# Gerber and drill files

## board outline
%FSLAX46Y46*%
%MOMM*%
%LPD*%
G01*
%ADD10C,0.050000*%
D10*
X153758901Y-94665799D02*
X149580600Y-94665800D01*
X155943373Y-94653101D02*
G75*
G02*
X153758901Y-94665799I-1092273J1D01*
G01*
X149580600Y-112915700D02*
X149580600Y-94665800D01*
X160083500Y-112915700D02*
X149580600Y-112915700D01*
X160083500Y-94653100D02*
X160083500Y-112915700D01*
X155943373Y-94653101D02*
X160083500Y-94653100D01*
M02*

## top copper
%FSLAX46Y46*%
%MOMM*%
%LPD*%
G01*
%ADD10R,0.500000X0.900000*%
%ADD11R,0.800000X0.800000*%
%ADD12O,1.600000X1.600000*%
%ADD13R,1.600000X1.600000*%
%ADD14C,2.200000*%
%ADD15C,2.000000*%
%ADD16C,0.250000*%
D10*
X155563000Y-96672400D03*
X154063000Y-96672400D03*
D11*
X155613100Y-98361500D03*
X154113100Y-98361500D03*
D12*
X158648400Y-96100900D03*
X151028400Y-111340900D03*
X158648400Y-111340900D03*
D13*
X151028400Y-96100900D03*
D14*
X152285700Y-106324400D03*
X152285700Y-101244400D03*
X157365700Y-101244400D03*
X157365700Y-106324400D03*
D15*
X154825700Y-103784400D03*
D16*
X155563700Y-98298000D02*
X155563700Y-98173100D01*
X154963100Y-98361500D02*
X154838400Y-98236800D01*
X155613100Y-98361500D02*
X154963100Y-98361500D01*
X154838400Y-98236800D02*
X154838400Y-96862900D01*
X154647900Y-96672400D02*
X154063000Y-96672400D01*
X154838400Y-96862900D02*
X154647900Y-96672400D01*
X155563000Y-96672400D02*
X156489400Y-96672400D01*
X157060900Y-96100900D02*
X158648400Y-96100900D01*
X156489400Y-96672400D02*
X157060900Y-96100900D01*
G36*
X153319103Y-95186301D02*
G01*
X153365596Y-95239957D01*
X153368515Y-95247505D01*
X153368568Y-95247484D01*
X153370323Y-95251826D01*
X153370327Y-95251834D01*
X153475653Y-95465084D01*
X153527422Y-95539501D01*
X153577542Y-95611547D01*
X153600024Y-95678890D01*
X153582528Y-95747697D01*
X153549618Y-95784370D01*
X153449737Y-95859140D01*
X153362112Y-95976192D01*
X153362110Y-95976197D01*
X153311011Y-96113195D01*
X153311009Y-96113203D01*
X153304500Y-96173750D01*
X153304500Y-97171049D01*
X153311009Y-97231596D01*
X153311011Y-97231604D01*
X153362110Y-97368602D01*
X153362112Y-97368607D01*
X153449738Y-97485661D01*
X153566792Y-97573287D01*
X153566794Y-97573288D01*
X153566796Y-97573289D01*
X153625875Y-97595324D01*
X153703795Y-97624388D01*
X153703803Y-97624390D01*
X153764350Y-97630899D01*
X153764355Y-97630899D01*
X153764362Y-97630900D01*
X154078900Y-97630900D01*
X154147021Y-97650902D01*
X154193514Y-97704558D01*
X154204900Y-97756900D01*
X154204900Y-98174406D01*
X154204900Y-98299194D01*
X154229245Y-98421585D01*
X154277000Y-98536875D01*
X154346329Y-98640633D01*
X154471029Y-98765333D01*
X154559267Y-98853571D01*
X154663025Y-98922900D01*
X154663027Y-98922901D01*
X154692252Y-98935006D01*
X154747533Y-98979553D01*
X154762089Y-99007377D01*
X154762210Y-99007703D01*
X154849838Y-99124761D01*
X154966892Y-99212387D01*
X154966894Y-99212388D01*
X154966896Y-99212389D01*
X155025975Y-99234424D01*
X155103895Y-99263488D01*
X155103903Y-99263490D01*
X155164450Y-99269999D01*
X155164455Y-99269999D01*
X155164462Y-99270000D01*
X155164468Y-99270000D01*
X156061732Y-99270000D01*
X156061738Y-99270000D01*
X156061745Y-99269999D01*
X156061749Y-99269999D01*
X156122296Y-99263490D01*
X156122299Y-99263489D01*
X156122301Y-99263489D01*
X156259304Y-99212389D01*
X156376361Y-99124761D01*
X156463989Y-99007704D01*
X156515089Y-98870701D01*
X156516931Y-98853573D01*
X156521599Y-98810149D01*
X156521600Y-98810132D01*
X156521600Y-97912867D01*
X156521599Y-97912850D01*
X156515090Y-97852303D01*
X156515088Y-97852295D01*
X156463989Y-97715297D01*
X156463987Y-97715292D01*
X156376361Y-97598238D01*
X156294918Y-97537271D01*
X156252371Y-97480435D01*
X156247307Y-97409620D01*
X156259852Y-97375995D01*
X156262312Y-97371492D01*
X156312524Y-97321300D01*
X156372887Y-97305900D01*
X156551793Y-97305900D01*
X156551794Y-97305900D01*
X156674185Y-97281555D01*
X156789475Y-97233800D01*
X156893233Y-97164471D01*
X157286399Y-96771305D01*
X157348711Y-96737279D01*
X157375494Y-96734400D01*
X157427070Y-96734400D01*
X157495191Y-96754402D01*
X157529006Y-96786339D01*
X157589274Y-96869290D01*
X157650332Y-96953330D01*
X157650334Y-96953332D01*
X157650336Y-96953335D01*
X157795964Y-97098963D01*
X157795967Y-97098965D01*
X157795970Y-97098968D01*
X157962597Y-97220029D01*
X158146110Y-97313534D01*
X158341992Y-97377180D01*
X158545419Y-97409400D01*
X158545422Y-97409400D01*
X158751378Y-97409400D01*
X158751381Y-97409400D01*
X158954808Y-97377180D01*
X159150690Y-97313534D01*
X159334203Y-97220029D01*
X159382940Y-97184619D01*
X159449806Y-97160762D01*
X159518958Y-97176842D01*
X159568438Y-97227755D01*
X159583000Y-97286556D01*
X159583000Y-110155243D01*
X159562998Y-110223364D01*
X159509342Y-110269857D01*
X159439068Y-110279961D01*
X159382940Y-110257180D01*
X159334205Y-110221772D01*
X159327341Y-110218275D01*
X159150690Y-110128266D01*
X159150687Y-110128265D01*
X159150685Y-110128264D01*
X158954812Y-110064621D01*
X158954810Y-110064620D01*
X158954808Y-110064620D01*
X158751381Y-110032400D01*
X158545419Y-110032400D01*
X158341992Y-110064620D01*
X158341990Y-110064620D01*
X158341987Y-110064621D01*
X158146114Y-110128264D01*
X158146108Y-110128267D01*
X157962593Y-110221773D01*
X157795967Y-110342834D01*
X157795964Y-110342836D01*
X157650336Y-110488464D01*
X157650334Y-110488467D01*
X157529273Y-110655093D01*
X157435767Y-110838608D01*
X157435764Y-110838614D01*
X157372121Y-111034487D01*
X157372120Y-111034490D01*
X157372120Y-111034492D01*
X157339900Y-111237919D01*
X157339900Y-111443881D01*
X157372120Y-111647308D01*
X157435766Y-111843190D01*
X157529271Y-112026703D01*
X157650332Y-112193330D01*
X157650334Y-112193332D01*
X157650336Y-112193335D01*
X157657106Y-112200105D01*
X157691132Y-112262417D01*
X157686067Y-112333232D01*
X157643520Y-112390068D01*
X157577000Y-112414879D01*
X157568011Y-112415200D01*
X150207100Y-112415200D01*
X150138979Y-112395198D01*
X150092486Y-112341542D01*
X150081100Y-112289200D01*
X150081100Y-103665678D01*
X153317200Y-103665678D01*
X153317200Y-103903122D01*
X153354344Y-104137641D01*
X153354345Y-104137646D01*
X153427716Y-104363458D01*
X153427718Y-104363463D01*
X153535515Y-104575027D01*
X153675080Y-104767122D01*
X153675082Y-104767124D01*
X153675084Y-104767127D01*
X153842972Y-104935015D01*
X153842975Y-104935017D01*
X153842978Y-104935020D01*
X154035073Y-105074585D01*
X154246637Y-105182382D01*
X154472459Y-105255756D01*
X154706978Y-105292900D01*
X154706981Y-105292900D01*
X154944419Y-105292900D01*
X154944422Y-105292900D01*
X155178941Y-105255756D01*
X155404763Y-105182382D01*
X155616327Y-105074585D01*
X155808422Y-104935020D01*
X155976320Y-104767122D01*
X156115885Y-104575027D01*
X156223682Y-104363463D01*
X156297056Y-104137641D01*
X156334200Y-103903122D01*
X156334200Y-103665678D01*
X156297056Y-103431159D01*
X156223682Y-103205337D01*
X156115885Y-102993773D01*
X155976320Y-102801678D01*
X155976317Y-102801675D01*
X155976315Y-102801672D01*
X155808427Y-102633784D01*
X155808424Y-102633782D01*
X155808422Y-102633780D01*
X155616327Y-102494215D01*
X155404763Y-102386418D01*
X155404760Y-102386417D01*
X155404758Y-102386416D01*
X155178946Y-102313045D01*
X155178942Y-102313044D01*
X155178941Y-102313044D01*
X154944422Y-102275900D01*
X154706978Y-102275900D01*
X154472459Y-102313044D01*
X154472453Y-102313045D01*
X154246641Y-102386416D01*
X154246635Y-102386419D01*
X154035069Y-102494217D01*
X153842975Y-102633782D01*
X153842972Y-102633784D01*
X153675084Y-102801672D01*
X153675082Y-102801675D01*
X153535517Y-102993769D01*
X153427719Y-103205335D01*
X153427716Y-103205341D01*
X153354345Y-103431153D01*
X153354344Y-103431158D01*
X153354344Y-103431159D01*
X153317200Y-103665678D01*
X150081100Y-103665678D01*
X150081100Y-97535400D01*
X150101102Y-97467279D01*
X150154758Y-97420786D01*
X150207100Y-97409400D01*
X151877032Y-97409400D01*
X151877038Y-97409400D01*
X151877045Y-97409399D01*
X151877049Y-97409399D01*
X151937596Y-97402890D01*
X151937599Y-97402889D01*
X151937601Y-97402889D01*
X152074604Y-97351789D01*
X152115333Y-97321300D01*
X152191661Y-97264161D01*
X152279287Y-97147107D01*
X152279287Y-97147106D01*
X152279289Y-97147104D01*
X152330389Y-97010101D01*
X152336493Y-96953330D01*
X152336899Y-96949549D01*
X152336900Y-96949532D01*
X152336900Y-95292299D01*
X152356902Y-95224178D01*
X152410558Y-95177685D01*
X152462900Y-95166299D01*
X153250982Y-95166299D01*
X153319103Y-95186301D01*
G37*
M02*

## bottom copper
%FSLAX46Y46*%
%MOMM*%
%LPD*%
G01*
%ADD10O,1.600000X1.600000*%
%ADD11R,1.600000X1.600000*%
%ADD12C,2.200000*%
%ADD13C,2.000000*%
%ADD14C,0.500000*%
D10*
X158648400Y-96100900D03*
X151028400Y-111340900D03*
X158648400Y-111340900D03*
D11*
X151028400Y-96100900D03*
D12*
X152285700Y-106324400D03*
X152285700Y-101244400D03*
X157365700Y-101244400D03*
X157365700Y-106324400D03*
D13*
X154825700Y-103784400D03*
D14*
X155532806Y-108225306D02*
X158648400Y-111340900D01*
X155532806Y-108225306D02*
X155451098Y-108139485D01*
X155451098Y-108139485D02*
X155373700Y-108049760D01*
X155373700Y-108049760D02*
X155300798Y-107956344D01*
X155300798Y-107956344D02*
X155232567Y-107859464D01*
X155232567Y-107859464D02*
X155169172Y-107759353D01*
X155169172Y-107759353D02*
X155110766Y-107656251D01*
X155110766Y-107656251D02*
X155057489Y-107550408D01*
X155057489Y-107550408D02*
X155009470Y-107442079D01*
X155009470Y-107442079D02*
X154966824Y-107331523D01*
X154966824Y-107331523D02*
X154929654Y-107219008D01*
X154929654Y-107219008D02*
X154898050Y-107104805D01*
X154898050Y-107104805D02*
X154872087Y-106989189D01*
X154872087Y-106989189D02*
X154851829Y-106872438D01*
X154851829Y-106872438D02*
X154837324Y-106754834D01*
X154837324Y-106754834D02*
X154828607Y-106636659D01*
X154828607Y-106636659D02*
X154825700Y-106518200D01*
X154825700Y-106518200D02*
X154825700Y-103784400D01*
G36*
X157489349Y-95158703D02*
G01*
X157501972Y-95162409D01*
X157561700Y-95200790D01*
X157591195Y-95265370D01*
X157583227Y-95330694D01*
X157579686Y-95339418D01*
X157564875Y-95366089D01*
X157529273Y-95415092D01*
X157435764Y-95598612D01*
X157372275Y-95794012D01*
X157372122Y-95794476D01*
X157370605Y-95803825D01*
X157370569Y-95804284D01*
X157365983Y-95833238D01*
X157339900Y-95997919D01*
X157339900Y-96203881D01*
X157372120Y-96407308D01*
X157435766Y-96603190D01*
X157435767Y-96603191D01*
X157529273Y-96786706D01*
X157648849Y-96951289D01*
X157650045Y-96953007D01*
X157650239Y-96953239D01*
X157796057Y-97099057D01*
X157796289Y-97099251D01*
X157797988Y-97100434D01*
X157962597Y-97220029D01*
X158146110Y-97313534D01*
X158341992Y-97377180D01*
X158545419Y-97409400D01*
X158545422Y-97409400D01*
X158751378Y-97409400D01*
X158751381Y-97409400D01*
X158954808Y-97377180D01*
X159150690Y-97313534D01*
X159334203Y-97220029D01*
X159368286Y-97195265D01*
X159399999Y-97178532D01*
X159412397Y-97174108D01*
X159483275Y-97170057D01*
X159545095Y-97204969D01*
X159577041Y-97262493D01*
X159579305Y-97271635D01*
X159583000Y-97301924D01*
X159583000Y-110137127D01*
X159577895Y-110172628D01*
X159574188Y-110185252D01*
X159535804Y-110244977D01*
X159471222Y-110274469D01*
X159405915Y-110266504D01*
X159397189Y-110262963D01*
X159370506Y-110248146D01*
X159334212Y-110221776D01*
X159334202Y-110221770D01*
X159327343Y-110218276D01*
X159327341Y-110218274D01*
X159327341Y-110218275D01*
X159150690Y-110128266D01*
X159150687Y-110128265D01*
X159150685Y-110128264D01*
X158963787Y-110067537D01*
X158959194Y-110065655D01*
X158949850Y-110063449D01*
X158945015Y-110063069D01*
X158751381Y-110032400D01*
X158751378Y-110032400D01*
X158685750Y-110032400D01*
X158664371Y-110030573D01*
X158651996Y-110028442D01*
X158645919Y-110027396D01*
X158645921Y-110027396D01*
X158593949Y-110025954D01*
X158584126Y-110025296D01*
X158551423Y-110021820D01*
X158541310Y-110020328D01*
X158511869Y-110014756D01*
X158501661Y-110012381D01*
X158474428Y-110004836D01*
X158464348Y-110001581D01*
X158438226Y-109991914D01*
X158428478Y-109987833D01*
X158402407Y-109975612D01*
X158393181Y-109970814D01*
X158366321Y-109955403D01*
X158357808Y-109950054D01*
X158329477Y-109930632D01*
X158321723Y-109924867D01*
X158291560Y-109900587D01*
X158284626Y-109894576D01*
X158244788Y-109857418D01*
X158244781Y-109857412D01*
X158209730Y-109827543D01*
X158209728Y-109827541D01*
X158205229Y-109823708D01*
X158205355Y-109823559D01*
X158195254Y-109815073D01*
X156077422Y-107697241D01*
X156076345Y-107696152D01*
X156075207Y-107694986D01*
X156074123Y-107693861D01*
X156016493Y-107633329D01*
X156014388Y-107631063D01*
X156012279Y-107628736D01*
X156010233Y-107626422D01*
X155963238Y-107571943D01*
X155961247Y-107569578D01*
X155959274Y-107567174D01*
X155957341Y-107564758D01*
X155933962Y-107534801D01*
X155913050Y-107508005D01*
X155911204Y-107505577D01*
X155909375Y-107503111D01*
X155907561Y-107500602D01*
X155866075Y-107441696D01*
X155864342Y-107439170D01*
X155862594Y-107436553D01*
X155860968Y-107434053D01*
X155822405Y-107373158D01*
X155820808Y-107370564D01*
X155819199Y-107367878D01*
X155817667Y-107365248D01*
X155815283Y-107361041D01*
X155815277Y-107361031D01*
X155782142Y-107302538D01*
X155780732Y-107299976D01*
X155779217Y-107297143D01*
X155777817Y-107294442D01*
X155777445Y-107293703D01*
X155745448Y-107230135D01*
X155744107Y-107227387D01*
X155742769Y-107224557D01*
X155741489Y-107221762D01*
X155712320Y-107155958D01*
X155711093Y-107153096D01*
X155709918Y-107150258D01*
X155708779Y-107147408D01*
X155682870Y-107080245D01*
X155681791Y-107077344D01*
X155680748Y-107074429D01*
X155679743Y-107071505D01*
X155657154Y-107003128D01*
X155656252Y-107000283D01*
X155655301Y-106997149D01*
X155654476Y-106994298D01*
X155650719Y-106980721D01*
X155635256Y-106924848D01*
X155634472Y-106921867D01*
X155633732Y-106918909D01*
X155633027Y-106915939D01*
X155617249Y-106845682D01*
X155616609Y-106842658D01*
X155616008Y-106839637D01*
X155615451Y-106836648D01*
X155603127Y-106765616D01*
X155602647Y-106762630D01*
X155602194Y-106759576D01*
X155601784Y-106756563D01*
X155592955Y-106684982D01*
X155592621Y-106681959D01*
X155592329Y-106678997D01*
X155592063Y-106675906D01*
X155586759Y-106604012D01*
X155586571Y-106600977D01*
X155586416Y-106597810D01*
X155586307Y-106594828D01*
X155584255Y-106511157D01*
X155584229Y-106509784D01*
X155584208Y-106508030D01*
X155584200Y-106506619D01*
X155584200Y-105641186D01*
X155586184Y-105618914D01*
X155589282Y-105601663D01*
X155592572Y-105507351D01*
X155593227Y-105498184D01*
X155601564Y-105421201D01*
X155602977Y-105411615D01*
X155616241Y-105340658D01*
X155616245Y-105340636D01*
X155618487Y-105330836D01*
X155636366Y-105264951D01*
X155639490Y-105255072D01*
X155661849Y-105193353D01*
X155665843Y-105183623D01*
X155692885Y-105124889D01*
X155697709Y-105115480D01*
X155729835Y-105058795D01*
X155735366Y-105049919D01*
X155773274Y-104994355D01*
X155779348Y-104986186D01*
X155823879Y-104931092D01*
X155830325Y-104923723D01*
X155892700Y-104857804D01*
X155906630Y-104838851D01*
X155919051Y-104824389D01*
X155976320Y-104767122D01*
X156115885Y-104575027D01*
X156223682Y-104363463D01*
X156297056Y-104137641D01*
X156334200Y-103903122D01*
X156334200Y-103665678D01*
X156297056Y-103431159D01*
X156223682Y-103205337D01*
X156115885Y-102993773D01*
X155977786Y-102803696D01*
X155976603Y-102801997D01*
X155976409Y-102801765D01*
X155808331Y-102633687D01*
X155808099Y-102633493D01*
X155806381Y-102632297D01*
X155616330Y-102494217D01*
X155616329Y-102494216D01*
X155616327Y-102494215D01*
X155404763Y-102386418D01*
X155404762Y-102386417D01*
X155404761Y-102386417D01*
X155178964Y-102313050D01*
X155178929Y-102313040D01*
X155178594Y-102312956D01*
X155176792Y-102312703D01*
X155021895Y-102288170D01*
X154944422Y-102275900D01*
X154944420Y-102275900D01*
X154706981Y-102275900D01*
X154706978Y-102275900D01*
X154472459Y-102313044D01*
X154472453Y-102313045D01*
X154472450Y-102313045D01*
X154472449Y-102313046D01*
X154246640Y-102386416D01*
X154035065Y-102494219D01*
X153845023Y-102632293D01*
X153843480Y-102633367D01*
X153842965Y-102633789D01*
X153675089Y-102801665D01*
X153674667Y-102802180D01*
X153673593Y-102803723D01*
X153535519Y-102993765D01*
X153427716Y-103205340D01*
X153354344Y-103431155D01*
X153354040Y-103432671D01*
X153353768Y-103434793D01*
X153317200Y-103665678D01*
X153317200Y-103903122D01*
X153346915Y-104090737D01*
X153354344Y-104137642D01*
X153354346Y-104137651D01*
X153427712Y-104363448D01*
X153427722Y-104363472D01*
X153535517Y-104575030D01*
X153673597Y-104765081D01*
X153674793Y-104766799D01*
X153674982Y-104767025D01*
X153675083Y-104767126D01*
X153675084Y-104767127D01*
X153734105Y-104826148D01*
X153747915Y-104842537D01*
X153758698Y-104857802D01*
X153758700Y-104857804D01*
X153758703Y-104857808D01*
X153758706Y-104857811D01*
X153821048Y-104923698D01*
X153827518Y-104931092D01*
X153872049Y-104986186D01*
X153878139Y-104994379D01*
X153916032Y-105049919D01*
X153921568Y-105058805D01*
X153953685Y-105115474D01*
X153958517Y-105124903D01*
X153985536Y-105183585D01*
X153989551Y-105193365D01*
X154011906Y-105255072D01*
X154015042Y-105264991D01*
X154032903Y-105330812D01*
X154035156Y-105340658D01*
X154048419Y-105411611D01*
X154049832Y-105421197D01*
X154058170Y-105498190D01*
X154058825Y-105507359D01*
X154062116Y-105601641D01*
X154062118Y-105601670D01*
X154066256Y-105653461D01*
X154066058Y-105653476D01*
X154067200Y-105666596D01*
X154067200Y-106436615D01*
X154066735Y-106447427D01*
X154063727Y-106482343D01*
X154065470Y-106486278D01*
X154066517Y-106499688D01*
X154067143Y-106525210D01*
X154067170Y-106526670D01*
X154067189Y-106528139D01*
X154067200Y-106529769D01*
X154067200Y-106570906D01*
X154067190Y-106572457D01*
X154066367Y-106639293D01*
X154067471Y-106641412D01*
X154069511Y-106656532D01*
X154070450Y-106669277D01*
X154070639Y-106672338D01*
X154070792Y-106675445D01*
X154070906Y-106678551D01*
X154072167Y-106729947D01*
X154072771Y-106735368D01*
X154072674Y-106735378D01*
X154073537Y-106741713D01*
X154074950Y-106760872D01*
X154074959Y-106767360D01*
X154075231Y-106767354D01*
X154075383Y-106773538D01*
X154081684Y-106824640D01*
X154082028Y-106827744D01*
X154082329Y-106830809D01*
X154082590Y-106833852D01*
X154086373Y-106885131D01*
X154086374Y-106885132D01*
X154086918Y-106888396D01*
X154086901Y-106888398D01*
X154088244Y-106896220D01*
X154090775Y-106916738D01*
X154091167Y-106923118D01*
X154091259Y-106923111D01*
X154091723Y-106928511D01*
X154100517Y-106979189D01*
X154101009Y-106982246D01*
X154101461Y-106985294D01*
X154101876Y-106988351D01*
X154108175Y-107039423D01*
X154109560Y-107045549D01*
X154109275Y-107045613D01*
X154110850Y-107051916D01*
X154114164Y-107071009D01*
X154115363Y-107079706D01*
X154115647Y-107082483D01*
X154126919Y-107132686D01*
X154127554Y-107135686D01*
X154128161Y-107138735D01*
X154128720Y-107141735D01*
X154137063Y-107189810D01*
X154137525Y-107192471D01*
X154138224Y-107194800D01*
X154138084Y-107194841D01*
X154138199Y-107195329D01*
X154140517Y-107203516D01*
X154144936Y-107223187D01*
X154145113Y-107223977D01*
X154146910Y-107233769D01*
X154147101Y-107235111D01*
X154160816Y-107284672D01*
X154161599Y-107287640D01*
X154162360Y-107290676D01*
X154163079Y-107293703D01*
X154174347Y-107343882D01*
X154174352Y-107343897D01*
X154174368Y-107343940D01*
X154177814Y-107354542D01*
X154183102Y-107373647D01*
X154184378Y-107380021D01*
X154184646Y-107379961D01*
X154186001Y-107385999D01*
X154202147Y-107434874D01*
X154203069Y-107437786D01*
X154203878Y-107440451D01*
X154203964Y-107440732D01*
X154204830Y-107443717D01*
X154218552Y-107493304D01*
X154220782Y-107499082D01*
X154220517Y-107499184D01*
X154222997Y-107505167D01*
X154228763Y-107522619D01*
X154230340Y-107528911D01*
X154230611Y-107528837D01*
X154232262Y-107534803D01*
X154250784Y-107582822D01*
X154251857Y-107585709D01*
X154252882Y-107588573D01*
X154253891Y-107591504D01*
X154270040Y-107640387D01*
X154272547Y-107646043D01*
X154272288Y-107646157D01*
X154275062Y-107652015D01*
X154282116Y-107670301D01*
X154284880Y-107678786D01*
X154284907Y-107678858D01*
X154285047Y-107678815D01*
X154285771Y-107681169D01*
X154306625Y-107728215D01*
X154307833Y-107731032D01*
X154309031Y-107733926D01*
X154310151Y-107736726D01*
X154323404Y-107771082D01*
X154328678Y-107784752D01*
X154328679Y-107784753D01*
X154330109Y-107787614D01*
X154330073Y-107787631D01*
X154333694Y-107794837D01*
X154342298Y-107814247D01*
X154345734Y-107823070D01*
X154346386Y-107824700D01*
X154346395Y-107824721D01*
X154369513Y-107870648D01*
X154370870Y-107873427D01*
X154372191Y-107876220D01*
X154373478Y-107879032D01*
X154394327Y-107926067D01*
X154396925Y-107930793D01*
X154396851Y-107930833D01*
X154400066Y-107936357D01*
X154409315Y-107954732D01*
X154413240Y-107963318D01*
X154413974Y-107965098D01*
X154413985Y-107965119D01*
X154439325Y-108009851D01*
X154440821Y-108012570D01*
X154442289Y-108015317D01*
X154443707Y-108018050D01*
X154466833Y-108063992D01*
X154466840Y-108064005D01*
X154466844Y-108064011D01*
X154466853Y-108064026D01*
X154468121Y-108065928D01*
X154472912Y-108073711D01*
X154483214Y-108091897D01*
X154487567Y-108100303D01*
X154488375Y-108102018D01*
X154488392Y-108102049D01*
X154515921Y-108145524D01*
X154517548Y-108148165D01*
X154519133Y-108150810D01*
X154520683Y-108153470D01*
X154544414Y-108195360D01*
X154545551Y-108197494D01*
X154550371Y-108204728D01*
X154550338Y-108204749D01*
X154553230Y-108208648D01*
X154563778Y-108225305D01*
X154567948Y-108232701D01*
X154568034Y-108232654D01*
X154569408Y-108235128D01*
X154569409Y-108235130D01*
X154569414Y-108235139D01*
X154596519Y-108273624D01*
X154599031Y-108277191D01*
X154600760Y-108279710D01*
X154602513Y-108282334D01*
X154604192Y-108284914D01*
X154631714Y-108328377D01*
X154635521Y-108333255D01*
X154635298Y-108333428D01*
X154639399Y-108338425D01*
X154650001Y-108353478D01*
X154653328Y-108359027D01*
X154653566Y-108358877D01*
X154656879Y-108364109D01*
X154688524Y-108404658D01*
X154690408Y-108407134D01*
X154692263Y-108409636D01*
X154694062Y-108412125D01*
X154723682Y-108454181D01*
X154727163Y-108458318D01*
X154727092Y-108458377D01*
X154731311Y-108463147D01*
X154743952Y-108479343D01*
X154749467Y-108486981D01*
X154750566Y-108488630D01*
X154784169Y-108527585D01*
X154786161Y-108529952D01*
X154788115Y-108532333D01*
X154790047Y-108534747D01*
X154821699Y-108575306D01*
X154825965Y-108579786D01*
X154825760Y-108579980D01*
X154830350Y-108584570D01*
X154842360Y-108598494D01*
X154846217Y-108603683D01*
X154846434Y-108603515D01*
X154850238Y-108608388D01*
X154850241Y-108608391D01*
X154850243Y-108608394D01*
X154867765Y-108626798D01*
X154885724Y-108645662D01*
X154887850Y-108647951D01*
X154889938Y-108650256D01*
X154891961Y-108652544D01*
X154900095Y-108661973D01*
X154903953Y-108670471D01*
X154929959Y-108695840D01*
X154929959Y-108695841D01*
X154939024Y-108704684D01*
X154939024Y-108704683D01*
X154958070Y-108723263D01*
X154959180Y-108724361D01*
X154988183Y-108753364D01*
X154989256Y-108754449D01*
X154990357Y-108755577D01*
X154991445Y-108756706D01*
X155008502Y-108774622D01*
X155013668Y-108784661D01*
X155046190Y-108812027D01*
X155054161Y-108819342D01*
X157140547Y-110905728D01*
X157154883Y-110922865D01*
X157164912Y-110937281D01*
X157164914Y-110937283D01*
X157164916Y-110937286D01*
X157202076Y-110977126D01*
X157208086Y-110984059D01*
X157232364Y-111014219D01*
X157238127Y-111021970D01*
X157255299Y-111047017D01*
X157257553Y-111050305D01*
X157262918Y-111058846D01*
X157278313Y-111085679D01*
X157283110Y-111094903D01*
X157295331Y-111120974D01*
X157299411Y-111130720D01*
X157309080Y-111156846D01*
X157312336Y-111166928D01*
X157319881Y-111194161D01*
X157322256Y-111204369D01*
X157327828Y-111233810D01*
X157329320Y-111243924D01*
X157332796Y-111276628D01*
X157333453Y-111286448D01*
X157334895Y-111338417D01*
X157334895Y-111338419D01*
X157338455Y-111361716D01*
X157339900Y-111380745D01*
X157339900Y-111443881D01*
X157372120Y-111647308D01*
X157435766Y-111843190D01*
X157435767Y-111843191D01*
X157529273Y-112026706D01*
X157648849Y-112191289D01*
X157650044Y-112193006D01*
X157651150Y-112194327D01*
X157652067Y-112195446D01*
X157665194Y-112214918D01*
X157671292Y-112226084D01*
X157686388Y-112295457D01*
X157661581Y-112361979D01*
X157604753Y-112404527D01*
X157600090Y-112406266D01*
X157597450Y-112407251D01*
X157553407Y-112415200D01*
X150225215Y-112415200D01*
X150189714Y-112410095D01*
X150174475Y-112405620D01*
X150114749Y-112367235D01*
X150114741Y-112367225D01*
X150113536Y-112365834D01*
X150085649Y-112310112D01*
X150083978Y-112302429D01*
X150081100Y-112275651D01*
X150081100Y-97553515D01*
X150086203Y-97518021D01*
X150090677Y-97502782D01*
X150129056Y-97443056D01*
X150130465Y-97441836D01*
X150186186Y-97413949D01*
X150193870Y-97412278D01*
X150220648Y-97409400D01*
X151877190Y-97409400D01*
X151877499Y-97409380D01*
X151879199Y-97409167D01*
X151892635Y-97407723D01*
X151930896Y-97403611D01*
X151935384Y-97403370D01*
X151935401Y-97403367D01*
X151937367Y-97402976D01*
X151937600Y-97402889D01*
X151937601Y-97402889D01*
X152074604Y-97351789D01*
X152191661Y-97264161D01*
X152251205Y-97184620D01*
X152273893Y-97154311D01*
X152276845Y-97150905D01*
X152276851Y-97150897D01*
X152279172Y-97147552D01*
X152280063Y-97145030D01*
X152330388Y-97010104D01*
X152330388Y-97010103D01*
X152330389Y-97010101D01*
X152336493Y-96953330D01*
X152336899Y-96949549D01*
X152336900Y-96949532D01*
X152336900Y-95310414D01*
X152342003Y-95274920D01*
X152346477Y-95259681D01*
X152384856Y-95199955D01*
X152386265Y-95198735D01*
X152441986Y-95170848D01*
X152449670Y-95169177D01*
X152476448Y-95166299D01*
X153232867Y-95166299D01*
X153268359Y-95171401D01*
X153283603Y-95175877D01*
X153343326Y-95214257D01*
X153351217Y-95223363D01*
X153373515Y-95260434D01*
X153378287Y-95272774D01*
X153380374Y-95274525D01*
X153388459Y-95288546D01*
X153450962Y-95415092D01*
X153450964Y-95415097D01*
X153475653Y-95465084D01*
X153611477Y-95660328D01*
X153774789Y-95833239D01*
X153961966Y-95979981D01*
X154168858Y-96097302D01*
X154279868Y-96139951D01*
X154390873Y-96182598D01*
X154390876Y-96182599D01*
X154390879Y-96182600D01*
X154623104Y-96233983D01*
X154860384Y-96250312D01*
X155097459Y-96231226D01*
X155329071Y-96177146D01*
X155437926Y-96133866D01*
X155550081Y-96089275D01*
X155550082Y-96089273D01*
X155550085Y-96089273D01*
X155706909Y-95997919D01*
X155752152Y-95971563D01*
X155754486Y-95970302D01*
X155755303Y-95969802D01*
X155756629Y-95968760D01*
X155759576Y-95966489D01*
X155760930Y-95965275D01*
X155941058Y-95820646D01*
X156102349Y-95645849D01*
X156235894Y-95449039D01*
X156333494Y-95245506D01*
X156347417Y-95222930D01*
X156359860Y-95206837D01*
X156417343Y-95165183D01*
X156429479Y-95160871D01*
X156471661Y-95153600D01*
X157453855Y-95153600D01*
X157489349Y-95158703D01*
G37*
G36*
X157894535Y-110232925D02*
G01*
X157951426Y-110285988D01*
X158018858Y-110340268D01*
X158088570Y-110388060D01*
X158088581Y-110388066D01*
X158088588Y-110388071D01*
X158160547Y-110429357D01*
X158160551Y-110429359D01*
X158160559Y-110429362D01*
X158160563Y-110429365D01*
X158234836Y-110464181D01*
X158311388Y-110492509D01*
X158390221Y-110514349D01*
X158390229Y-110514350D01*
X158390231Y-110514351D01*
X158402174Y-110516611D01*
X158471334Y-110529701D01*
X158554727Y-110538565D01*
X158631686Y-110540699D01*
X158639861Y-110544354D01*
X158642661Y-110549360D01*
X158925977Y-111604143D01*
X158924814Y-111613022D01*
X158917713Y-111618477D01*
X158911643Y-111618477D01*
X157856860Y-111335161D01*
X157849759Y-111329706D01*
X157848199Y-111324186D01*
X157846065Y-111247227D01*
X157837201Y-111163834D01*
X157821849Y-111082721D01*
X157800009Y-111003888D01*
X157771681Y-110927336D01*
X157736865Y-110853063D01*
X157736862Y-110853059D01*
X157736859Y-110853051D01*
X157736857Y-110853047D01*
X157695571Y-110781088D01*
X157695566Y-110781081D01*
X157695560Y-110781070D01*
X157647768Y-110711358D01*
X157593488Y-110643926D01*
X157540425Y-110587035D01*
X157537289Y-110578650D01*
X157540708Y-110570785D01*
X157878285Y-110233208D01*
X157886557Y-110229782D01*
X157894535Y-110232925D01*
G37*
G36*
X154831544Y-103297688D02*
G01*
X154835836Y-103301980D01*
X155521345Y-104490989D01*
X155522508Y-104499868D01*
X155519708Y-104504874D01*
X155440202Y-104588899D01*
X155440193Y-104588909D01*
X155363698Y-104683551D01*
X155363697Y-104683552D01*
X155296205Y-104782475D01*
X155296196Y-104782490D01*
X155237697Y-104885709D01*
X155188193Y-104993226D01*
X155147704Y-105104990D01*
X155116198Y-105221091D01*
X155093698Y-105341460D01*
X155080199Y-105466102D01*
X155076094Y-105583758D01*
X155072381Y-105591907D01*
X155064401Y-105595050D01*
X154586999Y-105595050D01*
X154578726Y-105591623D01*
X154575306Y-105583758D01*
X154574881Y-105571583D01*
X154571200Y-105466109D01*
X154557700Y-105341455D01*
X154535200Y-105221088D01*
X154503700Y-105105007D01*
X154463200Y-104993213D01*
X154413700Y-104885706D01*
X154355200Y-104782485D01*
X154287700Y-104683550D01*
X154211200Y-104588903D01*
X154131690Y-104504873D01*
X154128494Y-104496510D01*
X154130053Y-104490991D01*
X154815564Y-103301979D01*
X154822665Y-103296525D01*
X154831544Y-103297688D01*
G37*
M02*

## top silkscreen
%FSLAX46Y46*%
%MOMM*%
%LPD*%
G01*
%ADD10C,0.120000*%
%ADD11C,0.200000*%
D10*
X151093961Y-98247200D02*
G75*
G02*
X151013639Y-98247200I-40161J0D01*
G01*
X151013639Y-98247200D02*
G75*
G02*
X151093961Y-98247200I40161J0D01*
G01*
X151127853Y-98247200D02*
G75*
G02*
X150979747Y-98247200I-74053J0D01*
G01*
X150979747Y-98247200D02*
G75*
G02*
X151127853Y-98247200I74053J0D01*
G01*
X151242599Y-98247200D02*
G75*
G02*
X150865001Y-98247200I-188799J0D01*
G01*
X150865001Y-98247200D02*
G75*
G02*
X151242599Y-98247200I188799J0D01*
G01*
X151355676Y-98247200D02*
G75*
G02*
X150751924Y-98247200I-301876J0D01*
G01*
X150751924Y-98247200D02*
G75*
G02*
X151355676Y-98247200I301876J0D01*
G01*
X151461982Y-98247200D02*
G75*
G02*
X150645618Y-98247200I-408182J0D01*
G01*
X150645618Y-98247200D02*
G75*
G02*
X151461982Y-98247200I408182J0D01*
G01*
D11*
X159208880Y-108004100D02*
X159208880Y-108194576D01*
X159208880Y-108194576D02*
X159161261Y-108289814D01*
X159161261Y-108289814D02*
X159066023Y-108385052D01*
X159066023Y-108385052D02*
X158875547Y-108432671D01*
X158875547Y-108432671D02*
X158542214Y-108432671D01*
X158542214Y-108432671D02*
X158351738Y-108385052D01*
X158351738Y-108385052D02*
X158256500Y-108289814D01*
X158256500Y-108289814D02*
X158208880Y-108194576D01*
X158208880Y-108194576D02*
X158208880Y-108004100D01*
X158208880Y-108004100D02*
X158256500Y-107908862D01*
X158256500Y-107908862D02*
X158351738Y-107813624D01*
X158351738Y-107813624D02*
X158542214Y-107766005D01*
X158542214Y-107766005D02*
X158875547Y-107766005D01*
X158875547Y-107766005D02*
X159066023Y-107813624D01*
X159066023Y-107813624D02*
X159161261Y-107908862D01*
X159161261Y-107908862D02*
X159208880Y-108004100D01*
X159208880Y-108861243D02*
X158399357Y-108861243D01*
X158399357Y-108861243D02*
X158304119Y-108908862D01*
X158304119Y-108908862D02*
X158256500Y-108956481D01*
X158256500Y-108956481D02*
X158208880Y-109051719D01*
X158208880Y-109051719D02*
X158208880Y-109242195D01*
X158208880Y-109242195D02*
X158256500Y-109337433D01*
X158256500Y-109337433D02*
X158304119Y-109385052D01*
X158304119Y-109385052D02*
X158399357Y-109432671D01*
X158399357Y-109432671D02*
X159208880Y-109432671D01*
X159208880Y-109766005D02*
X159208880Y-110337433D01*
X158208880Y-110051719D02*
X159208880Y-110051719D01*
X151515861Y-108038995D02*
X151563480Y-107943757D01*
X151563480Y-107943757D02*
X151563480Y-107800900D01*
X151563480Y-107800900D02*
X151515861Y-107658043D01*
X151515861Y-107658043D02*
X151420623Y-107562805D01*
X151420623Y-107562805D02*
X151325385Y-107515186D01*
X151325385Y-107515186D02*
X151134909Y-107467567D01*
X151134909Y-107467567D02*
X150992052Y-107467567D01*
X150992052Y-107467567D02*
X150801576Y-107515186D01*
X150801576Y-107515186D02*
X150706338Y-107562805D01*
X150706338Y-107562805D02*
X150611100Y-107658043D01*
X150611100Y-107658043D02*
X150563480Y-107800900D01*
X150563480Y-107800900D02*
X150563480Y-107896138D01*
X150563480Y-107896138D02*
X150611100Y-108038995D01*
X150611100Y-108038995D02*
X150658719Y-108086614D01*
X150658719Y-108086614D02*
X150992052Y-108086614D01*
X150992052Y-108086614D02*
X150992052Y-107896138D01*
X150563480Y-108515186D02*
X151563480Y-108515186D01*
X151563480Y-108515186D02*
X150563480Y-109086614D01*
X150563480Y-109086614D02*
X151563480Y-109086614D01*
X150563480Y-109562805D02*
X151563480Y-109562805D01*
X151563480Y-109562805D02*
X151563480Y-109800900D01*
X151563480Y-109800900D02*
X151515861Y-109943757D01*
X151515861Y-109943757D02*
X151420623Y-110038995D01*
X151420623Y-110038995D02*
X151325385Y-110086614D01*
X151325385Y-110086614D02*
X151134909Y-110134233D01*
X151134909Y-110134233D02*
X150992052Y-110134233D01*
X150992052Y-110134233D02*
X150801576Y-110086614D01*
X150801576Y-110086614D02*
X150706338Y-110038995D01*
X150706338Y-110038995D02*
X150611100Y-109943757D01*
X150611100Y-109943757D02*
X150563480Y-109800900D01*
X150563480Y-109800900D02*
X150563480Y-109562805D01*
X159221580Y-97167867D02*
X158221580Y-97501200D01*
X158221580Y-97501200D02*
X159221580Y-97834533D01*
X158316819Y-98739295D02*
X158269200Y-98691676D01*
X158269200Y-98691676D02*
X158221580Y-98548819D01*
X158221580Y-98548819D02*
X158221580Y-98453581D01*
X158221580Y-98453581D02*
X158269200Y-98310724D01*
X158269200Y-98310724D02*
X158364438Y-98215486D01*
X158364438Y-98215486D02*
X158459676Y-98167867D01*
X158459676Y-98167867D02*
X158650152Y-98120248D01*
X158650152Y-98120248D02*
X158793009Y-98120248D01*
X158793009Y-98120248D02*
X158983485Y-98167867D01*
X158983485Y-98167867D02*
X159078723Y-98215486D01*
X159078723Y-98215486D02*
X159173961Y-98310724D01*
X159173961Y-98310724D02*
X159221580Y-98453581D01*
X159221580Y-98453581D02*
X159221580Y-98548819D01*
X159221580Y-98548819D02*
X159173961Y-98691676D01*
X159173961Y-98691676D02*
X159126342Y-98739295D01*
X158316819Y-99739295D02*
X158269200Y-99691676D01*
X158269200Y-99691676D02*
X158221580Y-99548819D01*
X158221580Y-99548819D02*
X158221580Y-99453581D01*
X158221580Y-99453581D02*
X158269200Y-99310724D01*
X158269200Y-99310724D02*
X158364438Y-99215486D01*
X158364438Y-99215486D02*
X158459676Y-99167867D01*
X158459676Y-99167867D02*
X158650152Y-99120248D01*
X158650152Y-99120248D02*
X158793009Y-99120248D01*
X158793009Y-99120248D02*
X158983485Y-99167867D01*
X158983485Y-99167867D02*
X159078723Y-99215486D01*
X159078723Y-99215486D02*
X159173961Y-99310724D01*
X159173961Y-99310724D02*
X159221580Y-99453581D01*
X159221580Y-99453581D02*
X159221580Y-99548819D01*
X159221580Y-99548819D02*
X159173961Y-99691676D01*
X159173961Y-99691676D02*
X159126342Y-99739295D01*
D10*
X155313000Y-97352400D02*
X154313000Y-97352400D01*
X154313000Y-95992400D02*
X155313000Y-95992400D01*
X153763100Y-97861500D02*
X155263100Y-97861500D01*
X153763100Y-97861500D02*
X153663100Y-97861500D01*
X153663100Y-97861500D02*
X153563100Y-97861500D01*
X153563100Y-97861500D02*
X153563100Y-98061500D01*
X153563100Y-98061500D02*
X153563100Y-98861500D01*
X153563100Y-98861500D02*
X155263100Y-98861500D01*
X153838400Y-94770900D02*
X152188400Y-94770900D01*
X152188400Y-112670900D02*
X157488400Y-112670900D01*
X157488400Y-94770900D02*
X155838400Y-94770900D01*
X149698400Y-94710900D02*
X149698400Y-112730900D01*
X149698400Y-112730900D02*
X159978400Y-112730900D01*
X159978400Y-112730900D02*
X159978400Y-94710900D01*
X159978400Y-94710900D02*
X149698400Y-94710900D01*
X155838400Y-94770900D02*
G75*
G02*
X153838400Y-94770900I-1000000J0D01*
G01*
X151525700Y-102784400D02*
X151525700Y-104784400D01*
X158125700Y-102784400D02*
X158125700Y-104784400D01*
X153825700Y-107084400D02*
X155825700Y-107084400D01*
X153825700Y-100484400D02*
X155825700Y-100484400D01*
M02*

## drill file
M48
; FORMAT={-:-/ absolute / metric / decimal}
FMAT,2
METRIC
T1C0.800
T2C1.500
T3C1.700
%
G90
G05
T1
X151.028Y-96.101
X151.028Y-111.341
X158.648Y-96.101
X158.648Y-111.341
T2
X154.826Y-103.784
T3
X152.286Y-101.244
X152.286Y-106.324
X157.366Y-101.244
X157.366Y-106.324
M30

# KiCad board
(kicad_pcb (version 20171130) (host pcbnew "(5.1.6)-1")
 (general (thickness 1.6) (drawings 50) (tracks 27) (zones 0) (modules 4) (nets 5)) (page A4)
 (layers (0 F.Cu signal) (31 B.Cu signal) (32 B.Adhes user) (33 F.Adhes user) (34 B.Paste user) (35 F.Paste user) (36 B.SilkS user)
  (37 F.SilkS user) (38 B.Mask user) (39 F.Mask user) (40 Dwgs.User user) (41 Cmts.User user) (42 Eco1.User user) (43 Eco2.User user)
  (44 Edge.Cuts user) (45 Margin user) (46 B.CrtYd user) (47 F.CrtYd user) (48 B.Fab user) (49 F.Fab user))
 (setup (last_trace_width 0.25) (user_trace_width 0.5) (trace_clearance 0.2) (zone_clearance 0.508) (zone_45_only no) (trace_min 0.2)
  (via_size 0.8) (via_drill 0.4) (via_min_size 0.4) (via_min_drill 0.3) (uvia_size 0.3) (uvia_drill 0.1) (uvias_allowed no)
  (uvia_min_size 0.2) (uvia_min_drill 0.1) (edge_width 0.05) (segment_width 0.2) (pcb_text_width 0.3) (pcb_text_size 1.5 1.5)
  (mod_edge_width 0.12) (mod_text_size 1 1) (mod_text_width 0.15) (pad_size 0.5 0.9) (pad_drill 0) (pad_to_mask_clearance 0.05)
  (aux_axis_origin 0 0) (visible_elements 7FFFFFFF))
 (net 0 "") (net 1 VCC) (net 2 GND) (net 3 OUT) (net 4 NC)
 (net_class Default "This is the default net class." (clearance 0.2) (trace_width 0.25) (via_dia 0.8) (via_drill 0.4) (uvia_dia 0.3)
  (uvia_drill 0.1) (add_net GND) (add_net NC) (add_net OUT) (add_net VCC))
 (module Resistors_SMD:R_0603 (layer F.Cu) (at 154.813 96.6724 180)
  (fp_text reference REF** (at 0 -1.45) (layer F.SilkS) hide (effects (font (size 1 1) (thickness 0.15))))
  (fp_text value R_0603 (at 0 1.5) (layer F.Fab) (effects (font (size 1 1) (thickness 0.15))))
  (fp_line (start -0.5 -0.68) (end 0.5 -0.68) (layer F.SilkS) (width 0.12))
  (fp_line (start 0.5 0.68) (end -0.5 0.68) (layer F.SilkS) (width 0.12))
  (pad 1 smd rect (at -0.75 0 180) (size 0.5 0.9) (layers F.Cu F.Paste F.Mask) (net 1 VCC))
  (pad 2 smd rect (at 0.75 0 180) (size 0.5 0.9) (layers F.Cu F.Paste F.Mask)))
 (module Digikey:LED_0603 (layer F.Cu) (at 154.8631 98.3615)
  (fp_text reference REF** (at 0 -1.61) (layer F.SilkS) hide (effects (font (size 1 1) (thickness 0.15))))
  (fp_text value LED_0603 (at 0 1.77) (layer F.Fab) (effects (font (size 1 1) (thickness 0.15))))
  (fp_line (start -1.1 -0.5) (end 0.4 -0.5) (layer F.SilkS) (width 0.12))
  (fp_line (start -1.1 -0.5) (end -1.2 -0.5) (layer F.SilkS) (width 0.12))
  (fp_line (start -1.2 -0.5) (end -1.3 -0.5) (layer F.SilkS) (width 0.12))
  (fp_line (start -1.3 -0.5) (end -1.3 -0.3) (layer F.SilkS) (width 0.12))
  (fp_line (start -1.3 -0.3) (end -1.3 0.5) (layer F.SilkS) (width 0.12))
  (fp_line (start -1.3 0.5) (end 0.4 0.5) (layer F.SilkS) (width 0.12))
  (pad 2 smd rect (at 0.75 0) (size 0.8 0.8) (layers F.Cu F.Paste F.Mask))
  (pad 1 smd rect (at -0.75 0) (size 0.8 0.8) (layers F.Cu F.Paste F.Mask) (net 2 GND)))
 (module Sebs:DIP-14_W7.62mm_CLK (layer F.Cu) (at 151.0284 96.1009)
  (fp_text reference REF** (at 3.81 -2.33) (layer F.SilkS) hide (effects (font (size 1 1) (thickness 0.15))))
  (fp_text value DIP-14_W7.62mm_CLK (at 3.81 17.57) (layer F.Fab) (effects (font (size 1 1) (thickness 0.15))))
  (fp_line (start 2.81 -1.33) (end 1.16 -1.33) (layer F.SilkS) (width 0.12))
  (fp_line (start 1.16 16.57) (end 6.46 16.57) (layer F.SilkS) (width 0.12))
  (fp_line (start 6.46 -1.33) (end 4.81 -1.33) (layer F.SilkS) (width 0.12))
  (fp_line (start -1.33 -1.39) (end -1.33 16.63) (layer F.SilkS) (width 0.12))
  (fp_line (start -1.33 16.63) (end 8.95 16.63) (layer F.SilkS) (width 0.12))
  (fp_line (start 8.95 16.63) (end 8.95 -1.39) (layer F.SilkS) (width 0.12))
  (fp_line (start 8.95 -1.39) (end -1.33 -1.39) (layer F.SilkS) (width 0.12))
  (fp_arc (start 3.81 -1.33) (end 2.81 -1.33) (angle -180) (layer F.SilkS) (width 0.12))
  (pad 14 thru_hole oval (at 7.62 0) (size 1.6 1.6) (drill 0.8) (layers *.Cu *.Mask) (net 1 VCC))
  (pad 7 thru_hole oval (at 0 15.24) (size 1.6 1.6) (drill 0.8) (layers *.Cu *.Mask) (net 2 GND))
  (pad 8 thru_hole oval (at 7.62 15.24) (size 1.6 1.6) (drill 0.8) (layers *.Cu *.Mask) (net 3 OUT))
  (pad 1 thru_hole rect (at 0 0) (size 1.6 1.6) (drill 0.8) (layers *.Cu *.Mask) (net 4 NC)))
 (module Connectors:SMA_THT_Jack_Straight (layer F.Cu) (at 154.8257 103.7844)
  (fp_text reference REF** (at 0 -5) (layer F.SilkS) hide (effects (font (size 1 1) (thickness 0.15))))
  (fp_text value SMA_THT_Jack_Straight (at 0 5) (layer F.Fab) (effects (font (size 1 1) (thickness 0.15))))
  (fp_line (start -3.3 -1) (end -3.3 1) (layer F.SilkS) (width 0.12))
  (fp_line (start 3.3 -1) (end 3.3 1) (layer F.SilkS) (width 0.12))
  (fp_line (start -1 3.3) (end 1 3.3) (layer F.SilkS) (width 0.12))
  (fp_line (start -1 -3.3) (end 1 -3.3) (layer F.SilkS) (width 0.12))
  (pad 2 thru_hole circle (at -2.54 2.54) (size 2.2 2.2) (drill 1.7) (layers *.Cu *.Mask) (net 2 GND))
  (pad 2 thru_hole circle (at -2.54 -2.54) (size 2.2 2.2) (drill 1.7) (layers *.Cu *.Mask) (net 2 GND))
  (pad 2 thru_hole circle (at 2.54 -2.54) (size 2.2 2.2) (drill 1.7) (layers *.Cu *.Mask) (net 2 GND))
  (pad 2 thru_hole circle (at 2.54 2.54) (size 2.2 2.2) (drill 1.7) (layers *.Cu *.Mask) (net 2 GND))
  (pad 1 thru_hole circle (at 0 0) (size 2 2) (drill 1.5) (layers *.Cu *.Mask) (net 3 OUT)))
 (gr_circle (center 151.0538 98.2472) (end 151.0665 98.2091) (layer F.SilkS) (width 0.12))
 (gr_circle (center 151.0538 98.2472) (end 151.0919 98.1837) (layer F.SilkS) (width 0.12))
 (gr_circle (center 151.0538 98.2472) (end 151.1173 98.0694) (layer F.SilkS) (width 0.12))
 (gr_circle (center 151.0538 98.2472) (end 151.13 97.9551) (layer F.SilkS) (width 0.12))
 (gr_circle (center 151.0538 98.2472) (end 151.461982 98.2472) (layer F.SilkS) (width 0.12))
 (gr_line (start 153.758901 94.665799) (end 149.5806 94.6658) (layer Edge.Cuts) (width 0.05))
 (gr_arc (start 154.8511 94.6531) (end 153.758901 94.665799) (angle -179.3338) (layer Edge.Cuts) (width 0.05))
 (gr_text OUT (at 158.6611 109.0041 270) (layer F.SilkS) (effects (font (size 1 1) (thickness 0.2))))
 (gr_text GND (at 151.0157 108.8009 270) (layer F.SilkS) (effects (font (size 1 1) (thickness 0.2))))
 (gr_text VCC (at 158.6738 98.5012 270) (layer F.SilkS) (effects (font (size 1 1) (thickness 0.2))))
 (gr_line (start 149.5806 112.9157) (end 149.5806 94.6658) (layer Edge.Cuts) (width 0.05))
 (gr_line (start 160.0835 112.9157) (end 149.5806 112.9157) (layer Edge.Cuts) (width 0.05))
 (gr_line (start 160.0835 94.6531) (end 160.0835 112.9157) (layer Edge.Cuts) (width 0.05))
 (gr_line (start 155.943373 94.653101) (end 160.0835 94.6531) (layer Edge.Cuts) (width 0.05))
 (segment (start 155.5637 98.298) (end 155.5637 98.1731) (width 0.25) (layer F.Cu) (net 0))
 (segment (start 154.9631 98.3615) (end 154.8384 98.2368) (width 0.25) (layer F.Cu) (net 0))
 (segment (start 155.6131 98.3615) (end 154.9631 98.3615) (width 0.25) (layer F.Cu) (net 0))
 (segment (start 154.8384 98.2368) (end 154.8384 96.8629) (width 0.25) (layer F.Cu) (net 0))
 (segment (start 154.6479 96.6724) (end 154.063 96.6724) (width 0.25) (layer F.Cu) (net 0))
 (segment (start 154.8384 96.8629) (end 154.6479 96.6724) (width 0.25) (layer F.Cu) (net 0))
 (segment (start 155.532806 108.225306) (end 158.6484 111.3409) (width 0.5) (layer B.Cu) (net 3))
 (segment (start 155.532806 108.225306) (end 155.451098 108.139485) (width 0.5) (layer B.Cu) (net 3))
 (segment (start 155.451098 108.139485) (end 155.3737 108.04976) (width 0.5) (layer B.Cu) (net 3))
 (segment (start 155.3737 108.04976) (end 155.300798 107.956344) (width 0.5) (layer B.Cu) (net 3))
 (segment (start 155.300798 107.956344) (end 155.232567 107.859464) (width 0.5) (layer B.Cu) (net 3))
 (segment (start 155.232567 107.859464) (end 155.169172 107.759353) (width 0.5) (layer B.Cu) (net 3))
 (segment (start 155.169172 107.759353) (end 155.110766 107.656251) (width 0.5) (layer B.Cu) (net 3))
 (segment (start 155.110766 107.656251) (end 155.057489 107.550408) (width 0.5) (layer B.Cu) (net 3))
 (segment (start 155.057489 107.550408) (end 155.00947 107.442079) (width 0.5) (layer B.Cu) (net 3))
 (segment (start 155.00947 107.442079) (end 154.966824 107.331523) (width 0.5) (layer B.Cu) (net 3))
 (segment (start 154.966824 107.331523) (end 154.929654 107.219008) (width 0.5) (layer B.Cu) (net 3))
 (segment (start 154.929654 107.219008) (end 154.89805 107.104805) (width 0.5) (layer B.Cu) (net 3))
 (segment (start 154.89805 107.104805) (end 154.872087 106.989189) (width 0.5) (layer B.Cu) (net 3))
 (segment (start 154.872087 106.989189) (end 154.851829 106.872438) (width 0.5) (layer B.Cu) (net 3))
 (segment (start 154.851829 106.872438) (end 154.837324 106.754834) (width 0.5) (layer B.Cu) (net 3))
 (segment (start 154.837324 106.754834) (end 154.828607 106.636659) (width 0.5) (layer B.Cu) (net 3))
 (segment (start 154.828607 106.636659) (end 154.8257 106.5182) (width 0.5) (layer B.Cu) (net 3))
 (segment (start 154.8257 106.5182) (end 154.8257 103.7844) (width 0.5) (layer B.Cu) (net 3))
 (segment (start 155.563 96.6724) (end 156.4894 96.6724) (width 0.25) (layer F.Cu) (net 1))
 (segment (start 157.0609 96.1009) (end 158.6484 96.1009) (width 0.25) (layer F.Cu) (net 1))
 (segment (start 156.4894 96.6724) (end 157.0609 96.1009) (width 0.25) (layer F.Cu) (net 1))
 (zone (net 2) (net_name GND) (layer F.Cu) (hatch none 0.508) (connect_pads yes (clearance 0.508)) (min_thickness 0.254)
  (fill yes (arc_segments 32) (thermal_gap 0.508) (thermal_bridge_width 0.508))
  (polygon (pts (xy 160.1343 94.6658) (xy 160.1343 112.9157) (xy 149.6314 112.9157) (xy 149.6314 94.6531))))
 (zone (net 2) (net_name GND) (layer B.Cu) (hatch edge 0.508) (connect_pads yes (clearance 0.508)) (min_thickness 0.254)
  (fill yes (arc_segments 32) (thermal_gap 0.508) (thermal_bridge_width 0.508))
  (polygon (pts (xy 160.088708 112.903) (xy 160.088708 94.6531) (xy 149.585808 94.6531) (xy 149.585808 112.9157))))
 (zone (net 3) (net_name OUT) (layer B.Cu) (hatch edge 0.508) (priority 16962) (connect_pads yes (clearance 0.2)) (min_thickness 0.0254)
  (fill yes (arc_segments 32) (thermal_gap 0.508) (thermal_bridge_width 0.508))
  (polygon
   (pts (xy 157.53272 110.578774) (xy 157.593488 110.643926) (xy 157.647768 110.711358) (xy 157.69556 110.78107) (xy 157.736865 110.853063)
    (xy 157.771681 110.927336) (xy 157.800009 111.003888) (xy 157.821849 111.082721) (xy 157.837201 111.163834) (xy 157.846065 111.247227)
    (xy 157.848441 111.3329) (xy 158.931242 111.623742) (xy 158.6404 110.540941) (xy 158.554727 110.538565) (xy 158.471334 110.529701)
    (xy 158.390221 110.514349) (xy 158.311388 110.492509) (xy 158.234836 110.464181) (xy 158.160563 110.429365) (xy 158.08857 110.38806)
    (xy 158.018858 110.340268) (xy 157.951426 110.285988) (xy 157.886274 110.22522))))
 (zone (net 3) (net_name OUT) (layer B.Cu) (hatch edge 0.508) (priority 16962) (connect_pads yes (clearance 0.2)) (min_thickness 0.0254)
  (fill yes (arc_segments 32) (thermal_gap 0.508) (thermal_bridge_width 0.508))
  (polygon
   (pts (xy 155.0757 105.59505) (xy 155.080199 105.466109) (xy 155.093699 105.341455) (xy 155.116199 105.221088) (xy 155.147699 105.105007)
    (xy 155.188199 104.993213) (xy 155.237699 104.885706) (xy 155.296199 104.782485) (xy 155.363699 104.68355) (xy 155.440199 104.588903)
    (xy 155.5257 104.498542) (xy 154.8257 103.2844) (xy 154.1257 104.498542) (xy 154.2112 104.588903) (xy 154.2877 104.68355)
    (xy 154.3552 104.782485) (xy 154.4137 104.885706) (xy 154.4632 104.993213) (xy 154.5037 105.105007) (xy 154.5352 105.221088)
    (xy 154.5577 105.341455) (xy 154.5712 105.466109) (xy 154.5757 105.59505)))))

